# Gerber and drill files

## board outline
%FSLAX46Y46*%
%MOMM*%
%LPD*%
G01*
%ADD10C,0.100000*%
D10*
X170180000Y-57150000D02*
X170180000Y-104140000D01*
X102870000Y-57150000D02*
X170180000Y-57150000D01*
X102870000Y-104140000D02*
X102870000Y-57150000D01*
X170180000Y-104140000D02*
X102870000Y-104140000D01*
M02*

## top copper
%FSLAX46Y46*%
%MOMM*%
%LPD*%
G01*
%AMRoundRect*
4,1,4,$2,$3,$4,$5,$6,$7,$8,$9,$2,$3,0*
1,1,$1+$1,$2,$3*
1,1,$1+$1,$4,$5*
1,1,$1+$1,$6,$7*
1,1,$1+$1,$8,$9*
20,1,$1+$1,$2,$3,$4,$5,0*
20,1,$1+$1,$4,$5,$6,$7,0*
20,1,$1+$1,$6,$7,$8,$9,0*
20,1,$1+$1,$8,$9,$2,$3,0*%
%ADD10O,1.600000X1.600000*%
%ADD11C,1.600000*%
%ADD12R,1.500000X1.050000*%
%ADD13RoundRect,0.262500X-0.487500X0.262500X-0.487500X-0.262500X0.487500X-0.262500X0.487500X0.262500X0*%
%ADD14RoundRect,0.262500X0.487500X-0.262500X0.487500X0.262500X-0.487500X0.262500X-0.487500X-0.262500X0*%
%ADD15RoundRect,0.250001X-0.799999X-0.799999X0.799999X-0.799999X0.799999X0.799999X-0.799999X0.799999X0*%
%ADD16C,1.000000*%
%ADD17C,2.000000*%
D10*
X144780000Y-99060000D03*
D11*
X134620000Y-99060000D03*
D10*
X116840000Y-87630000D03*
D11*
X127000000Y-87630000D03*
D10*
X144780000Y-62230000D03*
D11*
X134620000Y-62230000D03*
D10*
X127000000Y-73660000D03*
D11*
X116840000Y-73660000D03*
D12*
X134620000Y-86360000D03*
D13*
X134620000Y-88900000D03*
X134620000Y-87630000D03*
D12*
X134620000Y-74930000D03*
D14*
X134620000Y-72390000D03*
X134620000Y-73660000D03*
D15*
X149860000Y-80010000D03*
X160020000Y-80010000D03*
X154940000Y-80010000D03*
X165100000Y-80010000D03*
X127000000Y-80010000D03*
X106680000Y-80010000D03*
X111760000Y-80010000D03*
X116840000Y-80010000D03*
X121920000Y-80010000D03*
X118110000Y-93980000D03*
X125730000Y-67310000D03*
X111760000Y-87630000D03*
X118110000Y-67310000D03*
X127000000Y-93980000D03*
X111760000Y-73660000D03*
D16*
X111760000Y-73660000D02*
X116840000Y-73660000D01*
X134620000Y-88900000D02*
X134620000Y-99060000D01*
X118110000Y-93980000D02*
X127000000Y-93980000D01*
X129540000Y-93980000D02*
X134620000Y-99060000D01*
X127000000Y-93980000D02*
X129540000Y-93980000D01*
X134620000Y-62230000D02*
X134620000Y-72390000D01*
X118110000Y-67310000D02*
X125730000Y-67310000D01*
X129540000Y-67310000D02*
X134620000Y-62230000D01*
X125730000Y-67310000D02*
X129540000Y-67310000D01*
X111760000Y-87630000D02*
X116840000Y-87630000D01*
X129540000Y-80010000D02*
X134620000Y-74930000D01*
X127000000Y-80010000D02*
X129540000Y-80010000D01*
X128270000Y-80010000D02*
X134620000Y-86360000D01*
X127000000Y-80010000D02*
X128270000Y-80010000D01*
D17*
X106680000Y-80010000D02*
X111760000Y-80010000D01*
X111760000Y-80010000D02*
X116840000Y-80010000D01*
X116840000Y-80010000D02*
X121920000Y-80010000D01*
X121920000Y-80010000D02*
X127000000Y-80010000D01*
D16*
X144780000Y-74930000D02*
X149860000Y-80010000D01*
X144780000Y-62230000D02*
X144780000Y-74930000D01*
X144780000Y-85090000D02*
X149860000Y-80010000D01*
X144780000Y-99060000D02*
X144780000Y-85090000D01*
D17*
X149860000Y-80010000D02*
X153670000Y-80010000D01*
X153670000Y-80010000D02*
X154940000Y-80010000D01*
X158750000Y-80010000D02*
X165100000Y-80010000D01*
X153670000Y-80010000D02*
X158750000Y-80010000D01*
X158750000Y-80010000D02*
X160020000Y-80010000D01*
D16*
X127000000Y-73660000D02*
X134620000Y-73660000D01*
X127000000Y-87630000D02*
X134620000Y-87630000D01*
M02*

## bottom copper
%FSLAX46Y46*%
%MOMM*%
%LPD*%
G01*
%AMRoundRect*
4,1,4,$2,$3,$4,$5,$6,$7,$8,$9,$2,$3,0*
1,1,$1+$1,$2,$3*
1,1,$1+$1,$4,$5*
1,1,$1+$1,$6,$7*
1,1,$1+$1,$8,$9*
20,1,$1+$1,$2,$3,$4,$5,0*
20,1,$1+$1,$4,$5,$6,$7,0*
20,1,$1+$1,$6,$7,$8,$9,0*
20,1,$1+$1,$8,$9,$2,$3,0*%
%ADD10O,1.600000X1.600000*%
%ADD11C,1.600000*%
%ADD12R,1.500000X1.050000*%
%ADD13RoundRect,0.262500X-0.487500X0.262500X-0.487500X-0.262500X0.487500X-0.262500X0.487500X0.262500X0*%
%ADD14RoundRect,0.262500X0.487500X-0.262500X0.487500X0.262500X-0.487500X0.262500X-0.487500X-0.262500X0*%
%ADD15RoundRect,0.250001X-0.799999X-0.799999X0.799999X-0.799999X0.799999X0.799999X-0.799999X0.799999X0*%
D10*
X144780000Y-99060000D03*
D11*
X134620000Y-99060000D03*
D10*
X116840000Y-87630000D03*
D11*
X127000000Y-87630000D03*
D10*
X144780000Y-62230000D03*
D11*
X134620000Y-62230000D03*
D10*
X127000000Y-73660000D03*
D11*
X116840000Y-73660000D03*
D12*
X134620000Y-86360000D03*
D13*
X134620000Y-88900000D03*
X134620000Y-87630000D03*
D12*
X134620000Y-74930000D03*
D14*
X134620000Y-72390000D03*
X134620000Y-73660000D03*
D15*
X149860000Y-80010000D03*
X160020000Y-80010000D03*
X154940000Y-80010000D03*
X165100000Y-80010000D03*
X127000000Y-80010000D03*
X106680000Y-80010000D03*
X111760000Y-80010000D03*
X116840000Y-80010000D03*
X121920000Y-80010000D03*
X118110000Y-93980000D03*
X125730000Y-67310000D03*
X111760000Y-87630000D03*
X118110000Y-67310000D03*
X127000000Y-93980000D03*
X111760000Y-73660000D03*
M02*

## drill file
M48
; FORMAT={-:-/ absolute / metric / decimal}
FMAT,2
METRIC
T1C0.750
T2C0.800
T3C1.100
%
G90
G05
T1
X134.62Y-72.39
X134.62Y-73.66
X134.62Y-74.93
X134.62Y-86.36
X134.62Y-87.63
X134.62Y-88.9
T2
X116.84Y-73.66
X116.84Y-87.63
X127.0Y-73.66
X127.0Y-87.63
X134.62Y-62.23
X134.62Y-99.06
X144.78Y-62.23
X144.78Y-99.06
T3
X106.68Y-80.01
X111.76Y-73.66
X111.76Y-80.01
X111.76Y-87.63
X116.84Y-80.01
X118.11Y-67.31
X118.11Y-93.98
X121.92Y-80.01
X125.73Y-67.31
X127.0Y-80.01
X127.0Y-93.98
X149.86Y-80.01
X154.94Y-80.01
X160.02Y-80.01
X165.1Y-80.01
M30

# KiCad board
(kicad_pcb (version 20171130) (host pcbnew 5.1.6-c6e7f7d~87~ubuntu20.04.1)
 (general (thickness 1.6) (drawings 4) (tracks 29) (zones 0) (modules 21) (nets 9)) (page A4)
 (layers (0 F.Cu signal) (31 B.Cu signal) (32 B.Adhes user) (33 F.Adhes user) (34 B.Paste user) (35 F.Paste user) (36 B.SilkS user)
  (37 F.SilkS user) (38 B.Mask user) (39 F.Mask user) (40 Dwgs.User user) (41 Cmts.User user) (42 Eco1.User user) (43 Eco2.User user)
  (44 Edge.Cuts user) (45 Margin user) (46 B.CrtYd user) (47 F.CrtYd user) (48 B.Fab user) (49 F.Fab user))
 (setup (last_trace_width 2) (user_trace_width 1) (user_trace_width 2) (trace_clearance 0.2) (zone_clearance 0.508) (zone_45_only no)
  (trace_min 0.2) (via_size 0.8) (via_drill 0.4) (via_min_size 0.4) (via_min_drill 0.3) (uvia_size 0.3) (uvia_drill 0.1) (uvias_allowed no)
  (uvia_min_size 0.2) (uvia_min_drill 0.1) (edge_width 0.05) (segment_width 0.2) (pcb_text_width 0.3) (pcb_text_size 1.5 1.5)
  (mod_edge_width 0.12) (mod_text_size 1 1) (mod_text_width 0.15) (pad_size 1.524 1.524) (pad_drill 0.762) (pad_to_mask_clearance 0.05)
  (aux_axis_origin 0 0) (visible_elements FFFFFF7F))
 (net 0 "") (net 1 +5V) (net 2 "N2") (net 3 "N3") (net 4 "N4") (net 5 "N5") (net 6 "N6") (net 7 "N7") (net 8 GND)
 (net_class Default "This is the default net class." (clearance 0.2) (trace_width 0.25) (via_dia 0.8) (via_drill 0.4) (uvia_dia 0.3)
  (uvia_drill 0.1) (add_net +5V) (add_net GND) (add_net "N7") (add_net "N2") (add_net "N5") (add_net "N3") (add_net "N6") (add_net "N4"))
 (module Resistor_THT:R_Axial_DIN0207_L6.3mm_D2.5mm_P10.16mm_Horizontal (layer F.Cu) (at 134.62 99.06)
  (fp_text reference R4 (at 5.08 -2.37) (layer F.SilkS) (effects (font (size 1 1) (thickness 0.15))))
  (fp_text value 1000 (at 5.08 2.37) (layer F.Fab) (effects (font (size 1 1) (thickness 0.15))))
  (pad 2 thru_hole oval (at 10.16 0) (size 1.6 1.6) (drill 0.8) (layers *.Cu *.Mask) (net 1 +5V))
  (pad 1 thru_hole circle (at 0 0) (size 1.6 1.6) (drill 0.8) (layers *.Cu *.Mask) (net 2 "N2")))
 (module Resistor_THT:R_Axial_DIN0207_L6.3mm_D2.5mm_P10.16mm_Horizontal (layer F.Cu) (at 127 87.63 180)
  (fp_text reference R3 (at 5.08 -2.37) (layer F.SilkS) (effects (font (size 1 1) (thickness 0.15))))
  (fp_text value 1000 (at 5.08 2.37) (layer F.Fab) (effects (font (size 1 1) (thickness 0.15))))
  (pad 2 thru_hole oval (at 10.16 0 180) (size 1.6 1.6) (drill 0.8) (layers *.Cu *.Mask) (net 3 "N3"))
  (pad 1 thru_hole circle (at 0 0 180) (size 1.6 1.6) (drill 0.8) (layers *.Cu *.Mask) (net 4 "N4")))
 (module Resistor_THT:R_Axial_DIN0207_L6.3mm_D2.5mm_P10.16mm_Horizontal (layer F.Cu) (at 134.62 62.23)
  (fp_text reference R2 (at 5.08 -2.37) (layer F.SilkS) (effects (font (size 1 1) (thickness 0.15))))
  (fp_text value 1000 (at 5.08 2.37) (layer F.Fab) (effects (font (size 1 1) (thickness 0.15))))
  (pad 2 thru_hole oval (at 10.16 0) (size 1.6 1.6) (drill 0.8) (layers *.Cu *.Mask) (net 1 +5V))
  (pad 1 thru_hole circle (at 0 0) (size 1.6 1.6) (drill 0.8) (layers *.Cu *.Mask) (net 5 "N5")))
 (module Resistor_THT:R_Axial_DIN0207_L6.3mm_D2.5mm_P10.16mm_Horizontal (layer F.Cu) (at 116.84 73.66)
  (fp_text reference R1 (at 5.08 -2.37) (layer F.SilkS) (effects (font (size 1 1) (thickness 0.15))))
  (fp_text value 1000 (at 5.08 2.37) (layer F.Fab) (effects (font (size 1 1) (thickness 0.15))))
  (pad 2 thru_hole oval (at 10.16 0) (size 1.6 1.6) (drill 0.8) (layers *.Cu *.Mask) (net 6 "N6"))
  (pad 1 thru_hole circle (at 0 0) (size 1.6 1.6) (drill 0.8) (layers *.Cu *.Mask) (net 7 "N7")))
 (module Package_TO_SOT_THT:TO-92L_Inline (layer F.Cu) (at 134.62 86.36 270)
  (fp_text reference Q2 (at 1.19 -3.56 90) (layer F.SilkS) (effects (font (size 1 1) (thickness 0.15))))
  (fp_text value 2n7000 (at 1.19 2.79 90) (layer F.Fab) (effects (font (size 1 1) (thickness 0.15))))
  (pad 1 thru_hole rect (at 0 0 270) (size 1.05 1.5) (drill 0.75) (layers *.Cu *.Mask) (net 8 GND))
  (pad 3 thru_hole roundrect (at 2.54 0 270) (size 1.05 1.5) (drill 0.75) (layers *.Cu *.Mask) (roundrect_rratio 0.25) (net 2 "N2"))
  (pad 2 thru_hole roundrect (at 1.27 0 270) (size 1.05 1.5) (drill 0.75) (layers *.Cu *.Mask) (roundrect_rratio 0.25) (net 4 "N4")))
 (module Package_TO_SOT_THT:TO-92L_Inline (layer F.Cu) (at 134.62 74.93 90)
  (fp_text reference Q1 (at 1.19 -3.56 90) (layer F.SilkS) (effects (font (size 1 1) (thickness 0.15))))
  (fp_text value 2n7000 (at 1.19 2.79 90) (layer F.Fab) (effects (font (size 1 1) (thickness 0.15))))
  (pad 1 thru_hole rect (at 0 0 90) (size 1.05 1.5) (drill 0.75) (layers *.Cu *.Mask) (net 8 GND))
  (pad 3 thru_hole roundrect (at 2.54 0 90) (size 1.05 1.5) (drill 0.75) (layers *.Cu *.Mask) (roundrect_rratio 0.25) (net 5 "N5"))
  (pad 2 thru_hole roundrect (at 1.27 0 90) (size 1.05 1.5) (drill 0.75) (layers *.Cu *.Mask) (roundrect_rratio 0.25) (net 6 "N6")))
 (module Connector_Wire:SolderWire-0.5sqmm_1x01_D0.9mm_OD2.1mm (layer F.Cu) (at 149.86 80.01)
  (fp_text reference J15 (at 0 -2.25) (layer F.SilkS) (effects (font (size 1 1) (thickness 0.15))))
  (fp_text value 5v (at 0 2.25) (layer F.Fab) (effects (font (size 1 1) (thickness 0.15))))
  (pad 1 thru_hole roundrect (at 0 0) (size 2.1 2.1) (drill 1.1) (layers *.Cu *.Mask) (roundrect_rratio 0.119048) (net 1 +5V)))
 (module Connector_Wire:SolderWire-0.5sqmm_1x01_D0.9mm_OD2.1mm (layer F.Cu) (at 160.02 80.01)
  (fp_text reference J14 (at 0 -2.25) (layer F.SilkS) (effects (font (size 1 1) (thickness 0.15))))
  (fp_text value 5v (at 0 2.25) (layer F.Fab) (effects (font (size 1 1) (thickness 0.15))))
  (pad 1 thru_hole roundrect (at 0 0) (size 2.1 2.1) (drill 1.1) (layers *.Cu *.Mask) (roundrect_rratio 0.119048) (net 1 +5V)))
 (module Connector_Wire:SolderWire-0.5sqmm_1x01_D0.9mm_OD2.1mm (layer F.Cu) (at 154.94 80.01)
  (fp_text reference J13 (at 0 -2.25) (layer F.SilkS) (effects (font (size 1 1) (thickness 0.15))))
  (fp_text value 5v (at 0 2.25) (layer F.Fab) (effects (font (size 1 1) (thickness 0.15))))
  (pad 1 thru_hole roundrect (at 0 0) (size 2.1 2.1) (drill 1.1) (layers *.Cu *.Mask) (roundrect_rratio 0.119048) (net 1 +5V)))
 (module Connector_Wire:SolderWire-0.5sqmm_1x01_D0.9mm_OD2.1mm (layer F.Cu) (at 165.1 80.01)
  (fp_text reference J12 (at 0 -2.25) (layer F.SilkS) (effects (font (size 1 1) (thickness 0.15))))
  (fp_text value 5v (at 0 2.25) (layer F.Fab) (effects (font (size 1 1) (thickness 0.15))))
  (pad 1 thru_hole roundrect (at 0 0) (size 2.1 2.1) (drill 1.1) (layers *.Cu *.Mask) (roundrect_rratio 0.119048) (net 1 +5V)))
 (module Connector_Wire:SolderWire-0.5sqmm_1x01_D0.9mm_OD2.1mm (layer F.Cu) (at 127 80.01)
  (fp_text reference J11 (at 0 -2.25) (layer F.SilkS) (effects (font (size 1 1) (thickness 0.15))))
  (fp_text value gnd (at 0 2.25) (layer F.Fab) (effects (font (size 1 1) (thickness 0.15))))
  (pad 1 thru_hole roundrect (at 0 0) (size 2.1 2.1) (drill 1.1) (layers *.Cu *.Mask) (roundrect_rratio 0.119048) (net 8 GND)))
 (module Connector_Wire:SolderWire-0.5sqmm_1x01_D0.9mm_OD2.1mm (layer F.Cu) (at 106.68 80.01)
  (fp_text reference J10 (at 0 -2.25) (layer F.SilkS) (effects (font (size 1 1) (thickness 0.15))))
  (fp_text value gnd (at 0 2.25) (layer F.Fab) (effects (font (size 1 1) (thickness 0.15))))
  (pad 1 thru_hole roundrect (at 0 0) (size 2.1 2.1) (drill 1.1) (layers *.Cu *.Mask) (roundrect_rratio 0.119048) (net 8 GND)))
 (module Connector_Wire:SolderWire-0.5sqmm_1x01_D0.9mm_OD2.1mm (layer F.Cu) (at 111.76 80.01)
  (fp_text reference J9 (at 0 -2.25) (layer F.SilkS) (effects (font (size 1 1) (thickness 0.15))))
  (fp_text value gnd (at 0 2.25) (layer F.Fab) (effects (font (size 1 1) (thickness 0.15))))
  (pad 1 thru_hole roundrect (at 0 0) (size 2.1 2.1) (drill 1.1) (layers *.Cu *.Mask) (roundrect_rratio 0.119048) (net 8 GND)))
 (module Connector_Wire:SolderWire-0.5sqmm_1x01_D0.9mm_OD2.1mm (layer F.Cu) (at 116.84 80.01)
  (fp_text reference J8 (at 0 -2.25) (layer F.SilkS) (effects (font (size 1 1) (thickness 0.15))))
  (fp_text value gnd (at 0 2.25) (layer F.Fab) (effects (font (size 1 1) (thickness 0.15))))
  (pad 1 thru_hole roundrect (at 0 0) (size 2.1 2.1) (drill 1.1) (layers *.Cu *.Mask) (roundrect_rratio 0.119048) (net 8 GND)))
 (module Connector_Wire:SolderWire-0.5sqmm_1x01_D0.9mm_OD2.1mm (layer F.Cu) (at 121.92 80.01)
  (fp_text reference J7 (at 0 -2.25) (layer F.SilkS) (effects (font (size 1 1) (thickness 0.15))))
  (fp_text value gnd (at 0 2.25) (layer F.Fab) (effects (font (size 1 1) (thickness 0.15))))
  (pad 1 thru_hole roundrect (at 0 0) (size 2.1 2.1) (drill 1.1) (layers *.Cu *.Mask) (roundrect_rratio 0.119048) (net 8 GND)))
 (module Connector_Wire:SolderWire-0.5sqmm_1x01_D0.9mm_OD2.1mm (layer F.Cu) (at 118.11 93.98)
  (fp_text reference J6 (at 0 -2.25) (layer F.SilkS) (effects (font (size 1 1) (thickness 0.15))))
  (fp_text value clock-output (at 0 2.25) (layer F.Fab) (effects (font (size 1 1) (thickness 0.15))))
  (pad 1 thru_hole roundrect (at 0 0) (size 2.1 2.1) (drill 1.1) (layers *.Cu *.Mask) (roundrect_rratio 0.119048) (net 2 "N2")))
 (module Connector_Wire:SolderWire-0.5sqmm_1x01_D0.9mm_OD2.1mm (layer F.Cu) (at 125.73 67.31)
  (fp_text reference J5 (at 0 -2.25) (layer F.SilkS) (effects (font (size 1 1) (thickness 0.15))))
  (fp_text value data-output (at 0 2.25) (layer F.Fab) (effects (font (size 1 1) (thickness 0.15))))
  (pad 1 thru_hole roundrect (at 0 0) (size 2.1 2.1) (drill 1.1) (layers *.Cu *.Mask) (roundrect_rratio 0.119048) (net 5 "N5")))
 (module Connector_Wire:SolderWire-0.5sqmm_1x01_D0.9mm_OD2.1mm (layer F.Cu) (at 111.76 87.63)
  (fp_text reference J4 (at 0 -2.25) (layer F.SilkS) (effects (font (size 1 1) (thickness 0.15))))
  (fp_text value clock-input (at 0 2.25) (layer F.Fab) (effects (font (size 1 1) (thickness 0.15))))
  (pad 1 thru_hole roundrect (at 0 0) (size 2.1 2.1) (drill 1.1) (layers *.Cu *.Mask) (roundrect_rratio 0.119048) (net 3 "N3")))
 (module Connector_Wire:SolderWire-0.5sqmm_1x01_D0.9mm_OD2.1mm (layer F.Cu) (at 118.11 67.31)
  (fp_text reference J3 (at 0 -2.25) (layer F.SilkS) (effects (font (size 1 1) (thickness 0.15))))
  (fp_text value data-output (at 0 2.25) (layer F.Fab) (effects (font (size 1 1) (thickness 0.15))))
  (pad 1 thru_hole roundrect (at 0 0) (size 2.1 2.1) (drill 1.1) (layers *.Cu *.Mask) (roundrect_rratio 0.119048) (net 5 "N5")))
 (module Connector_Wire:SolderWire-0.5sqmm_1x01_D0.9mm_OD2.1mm (layer F.Cu) (at 127 93.98)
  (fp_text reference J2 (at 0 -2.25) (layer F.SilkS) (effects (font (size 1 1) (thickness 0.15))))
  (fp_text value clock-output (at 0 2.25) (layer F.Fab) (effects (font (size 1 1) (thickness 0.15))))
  (pad 1 thru_hole roundrect (at 0 0) (size 2.1 2.1) (drill 1.1) (layers *.Cu *.Mask) (roundrect_rratio 0.119048) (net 2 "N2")))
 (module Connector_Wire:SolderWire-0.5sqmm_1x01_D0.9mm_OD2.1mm (layer F.Cu) (at 111.76 73.66)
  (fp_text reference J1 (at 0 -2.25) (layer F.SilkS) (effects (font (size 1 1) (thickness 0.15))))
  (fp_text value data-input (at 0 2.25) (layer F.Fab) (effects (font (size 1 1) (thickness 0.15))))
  (pad 1 thru_hole roundrect (at 0 0) (size 2.1 2.1) (drill 1.1) (layers *.Cu *.Mask) (roundrect_rratio 0.119048) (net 7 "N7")))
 (gr_line (start 170.18 57.15) (end 170.18 104.14) (layer Edge.Cuts) (width 0.1))
 (gr_line (start 102.87 57.15) (end 170.18 57.15) (layer Edge.Cuts) (width 0.1))
 (gr_line (start 102.87 104.14) (end 102.87 57.15) (layer Edge.Cuts) (width 0.1))
 (gr_line (start 170.18 104.14) (end 102.87 104.14) (layer Edge.Cuts) (width 0.1))
 (segment (start 111.76 73.66) (end 116.84 73.66) (width 1) (layer F.Cu) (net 7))
 (segment (start 134.62 88.9) (end 134.62 99.06) (width 1) (layer F.Cu) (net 2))
 (segment (start 118.11 93.98) (end 127 93.98) (width 1) (layer F.Cu) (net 2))
 (segment (start 129.54 93.98) (end 134.62 99.06) (width 1) (layer F.Cu) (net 2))
 (segment (start 127 93.98) (end 129.54 93.98) (width 1) (layer F.Cu) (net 2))
 (segment (start 134.62 62.23) (end 134.62 72.39) (width 1) (layer F.Cu) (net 5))
 (segment (start 118.11 67.31) (end 125.73 67.31) (width 1) (layer F.Cu) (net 5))
 (segment (start 129.54 67.31) (end 134.62 62.23) (width 1) (layer F.Cu) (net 5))
 (segment (start 125.73 67.31) (end 129.54 67.31) (width 1) (layer F.Cu) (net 5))
 (segment (start 111.76 87.63) (end 116.84 87.63) (width 1) (layer F.Cu) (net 3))
 (segment (start 129.54 80.01) (end 134.62 74.93) (width 1) (layer F.Cu) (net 8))
 (segment (start 127 80.01) (end 129.54 80.01) (width 1) (layer F.Cu) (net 8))
 (segment (start 128.27 80.01) (end 134.62 86.36) (width 1) (layer F.Cu) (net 8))
 (segment (start 127 80.01) (end 128.27 80.01) (width 1) (layer F.Cu) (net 8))
 (segment (start 106.68 80.01) (end 111.76 80.01) (width 2) (layer F.Cu) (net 8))
 (segment (start 111.76 80.01) (end 116.84 80.01) (width 2) (layer F.Cu) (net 8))
 (segment (start 116.84 80.01) (end 121.92 80.01) (width 2) (layer F.Cu) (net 8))
 (segment (start 121.92 80.01) (end 127 80.01) (width 2) (layer F.Cu) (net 8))
 (segment (start 144.78 74.93) (end 149.86 80.01) (width 1) (layer F.Cu) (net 1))
 (segment (start 144.78 62.23) (end 144.78 74.93) (width 1) (layer F.Cu) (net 1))
 (segment (start 144.78 85.09) (end 149.86 80.01) (width 1) (layer F.Cu) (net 1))
 (segment (start 144.78 99.06) (end 144.78 85.09) (width 1) (layer F.Cu) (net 1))
 (segment (start 149.86 80.01) (end 153.67 80.01) (width 2) (layer F.Cu) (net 1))
 (segment (start 153.67 80.01) (end 154.94 80.01) (width 2) (layer F.Cu) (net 1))
 (segment (start 158.75 80.01) (end 165.1 80.01) (width 2) (layer F.Cu) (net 1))
 (segment (start 153.67 80.01) (end 158.75 80.01) (width 2) (layer F.Cu) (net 1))
 (segment (start 158.75 80.01) (end 160.02 80.01) (width 2) (layer F.Cu) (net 1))
 (segment (start 127 73.66) (end 134.62 73.66) (width 1) (layer F.Cu) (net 6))
 (segment (start 127 87.63) (end 134.62 87.63) (width 1) (layer F.Cu) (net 4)))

